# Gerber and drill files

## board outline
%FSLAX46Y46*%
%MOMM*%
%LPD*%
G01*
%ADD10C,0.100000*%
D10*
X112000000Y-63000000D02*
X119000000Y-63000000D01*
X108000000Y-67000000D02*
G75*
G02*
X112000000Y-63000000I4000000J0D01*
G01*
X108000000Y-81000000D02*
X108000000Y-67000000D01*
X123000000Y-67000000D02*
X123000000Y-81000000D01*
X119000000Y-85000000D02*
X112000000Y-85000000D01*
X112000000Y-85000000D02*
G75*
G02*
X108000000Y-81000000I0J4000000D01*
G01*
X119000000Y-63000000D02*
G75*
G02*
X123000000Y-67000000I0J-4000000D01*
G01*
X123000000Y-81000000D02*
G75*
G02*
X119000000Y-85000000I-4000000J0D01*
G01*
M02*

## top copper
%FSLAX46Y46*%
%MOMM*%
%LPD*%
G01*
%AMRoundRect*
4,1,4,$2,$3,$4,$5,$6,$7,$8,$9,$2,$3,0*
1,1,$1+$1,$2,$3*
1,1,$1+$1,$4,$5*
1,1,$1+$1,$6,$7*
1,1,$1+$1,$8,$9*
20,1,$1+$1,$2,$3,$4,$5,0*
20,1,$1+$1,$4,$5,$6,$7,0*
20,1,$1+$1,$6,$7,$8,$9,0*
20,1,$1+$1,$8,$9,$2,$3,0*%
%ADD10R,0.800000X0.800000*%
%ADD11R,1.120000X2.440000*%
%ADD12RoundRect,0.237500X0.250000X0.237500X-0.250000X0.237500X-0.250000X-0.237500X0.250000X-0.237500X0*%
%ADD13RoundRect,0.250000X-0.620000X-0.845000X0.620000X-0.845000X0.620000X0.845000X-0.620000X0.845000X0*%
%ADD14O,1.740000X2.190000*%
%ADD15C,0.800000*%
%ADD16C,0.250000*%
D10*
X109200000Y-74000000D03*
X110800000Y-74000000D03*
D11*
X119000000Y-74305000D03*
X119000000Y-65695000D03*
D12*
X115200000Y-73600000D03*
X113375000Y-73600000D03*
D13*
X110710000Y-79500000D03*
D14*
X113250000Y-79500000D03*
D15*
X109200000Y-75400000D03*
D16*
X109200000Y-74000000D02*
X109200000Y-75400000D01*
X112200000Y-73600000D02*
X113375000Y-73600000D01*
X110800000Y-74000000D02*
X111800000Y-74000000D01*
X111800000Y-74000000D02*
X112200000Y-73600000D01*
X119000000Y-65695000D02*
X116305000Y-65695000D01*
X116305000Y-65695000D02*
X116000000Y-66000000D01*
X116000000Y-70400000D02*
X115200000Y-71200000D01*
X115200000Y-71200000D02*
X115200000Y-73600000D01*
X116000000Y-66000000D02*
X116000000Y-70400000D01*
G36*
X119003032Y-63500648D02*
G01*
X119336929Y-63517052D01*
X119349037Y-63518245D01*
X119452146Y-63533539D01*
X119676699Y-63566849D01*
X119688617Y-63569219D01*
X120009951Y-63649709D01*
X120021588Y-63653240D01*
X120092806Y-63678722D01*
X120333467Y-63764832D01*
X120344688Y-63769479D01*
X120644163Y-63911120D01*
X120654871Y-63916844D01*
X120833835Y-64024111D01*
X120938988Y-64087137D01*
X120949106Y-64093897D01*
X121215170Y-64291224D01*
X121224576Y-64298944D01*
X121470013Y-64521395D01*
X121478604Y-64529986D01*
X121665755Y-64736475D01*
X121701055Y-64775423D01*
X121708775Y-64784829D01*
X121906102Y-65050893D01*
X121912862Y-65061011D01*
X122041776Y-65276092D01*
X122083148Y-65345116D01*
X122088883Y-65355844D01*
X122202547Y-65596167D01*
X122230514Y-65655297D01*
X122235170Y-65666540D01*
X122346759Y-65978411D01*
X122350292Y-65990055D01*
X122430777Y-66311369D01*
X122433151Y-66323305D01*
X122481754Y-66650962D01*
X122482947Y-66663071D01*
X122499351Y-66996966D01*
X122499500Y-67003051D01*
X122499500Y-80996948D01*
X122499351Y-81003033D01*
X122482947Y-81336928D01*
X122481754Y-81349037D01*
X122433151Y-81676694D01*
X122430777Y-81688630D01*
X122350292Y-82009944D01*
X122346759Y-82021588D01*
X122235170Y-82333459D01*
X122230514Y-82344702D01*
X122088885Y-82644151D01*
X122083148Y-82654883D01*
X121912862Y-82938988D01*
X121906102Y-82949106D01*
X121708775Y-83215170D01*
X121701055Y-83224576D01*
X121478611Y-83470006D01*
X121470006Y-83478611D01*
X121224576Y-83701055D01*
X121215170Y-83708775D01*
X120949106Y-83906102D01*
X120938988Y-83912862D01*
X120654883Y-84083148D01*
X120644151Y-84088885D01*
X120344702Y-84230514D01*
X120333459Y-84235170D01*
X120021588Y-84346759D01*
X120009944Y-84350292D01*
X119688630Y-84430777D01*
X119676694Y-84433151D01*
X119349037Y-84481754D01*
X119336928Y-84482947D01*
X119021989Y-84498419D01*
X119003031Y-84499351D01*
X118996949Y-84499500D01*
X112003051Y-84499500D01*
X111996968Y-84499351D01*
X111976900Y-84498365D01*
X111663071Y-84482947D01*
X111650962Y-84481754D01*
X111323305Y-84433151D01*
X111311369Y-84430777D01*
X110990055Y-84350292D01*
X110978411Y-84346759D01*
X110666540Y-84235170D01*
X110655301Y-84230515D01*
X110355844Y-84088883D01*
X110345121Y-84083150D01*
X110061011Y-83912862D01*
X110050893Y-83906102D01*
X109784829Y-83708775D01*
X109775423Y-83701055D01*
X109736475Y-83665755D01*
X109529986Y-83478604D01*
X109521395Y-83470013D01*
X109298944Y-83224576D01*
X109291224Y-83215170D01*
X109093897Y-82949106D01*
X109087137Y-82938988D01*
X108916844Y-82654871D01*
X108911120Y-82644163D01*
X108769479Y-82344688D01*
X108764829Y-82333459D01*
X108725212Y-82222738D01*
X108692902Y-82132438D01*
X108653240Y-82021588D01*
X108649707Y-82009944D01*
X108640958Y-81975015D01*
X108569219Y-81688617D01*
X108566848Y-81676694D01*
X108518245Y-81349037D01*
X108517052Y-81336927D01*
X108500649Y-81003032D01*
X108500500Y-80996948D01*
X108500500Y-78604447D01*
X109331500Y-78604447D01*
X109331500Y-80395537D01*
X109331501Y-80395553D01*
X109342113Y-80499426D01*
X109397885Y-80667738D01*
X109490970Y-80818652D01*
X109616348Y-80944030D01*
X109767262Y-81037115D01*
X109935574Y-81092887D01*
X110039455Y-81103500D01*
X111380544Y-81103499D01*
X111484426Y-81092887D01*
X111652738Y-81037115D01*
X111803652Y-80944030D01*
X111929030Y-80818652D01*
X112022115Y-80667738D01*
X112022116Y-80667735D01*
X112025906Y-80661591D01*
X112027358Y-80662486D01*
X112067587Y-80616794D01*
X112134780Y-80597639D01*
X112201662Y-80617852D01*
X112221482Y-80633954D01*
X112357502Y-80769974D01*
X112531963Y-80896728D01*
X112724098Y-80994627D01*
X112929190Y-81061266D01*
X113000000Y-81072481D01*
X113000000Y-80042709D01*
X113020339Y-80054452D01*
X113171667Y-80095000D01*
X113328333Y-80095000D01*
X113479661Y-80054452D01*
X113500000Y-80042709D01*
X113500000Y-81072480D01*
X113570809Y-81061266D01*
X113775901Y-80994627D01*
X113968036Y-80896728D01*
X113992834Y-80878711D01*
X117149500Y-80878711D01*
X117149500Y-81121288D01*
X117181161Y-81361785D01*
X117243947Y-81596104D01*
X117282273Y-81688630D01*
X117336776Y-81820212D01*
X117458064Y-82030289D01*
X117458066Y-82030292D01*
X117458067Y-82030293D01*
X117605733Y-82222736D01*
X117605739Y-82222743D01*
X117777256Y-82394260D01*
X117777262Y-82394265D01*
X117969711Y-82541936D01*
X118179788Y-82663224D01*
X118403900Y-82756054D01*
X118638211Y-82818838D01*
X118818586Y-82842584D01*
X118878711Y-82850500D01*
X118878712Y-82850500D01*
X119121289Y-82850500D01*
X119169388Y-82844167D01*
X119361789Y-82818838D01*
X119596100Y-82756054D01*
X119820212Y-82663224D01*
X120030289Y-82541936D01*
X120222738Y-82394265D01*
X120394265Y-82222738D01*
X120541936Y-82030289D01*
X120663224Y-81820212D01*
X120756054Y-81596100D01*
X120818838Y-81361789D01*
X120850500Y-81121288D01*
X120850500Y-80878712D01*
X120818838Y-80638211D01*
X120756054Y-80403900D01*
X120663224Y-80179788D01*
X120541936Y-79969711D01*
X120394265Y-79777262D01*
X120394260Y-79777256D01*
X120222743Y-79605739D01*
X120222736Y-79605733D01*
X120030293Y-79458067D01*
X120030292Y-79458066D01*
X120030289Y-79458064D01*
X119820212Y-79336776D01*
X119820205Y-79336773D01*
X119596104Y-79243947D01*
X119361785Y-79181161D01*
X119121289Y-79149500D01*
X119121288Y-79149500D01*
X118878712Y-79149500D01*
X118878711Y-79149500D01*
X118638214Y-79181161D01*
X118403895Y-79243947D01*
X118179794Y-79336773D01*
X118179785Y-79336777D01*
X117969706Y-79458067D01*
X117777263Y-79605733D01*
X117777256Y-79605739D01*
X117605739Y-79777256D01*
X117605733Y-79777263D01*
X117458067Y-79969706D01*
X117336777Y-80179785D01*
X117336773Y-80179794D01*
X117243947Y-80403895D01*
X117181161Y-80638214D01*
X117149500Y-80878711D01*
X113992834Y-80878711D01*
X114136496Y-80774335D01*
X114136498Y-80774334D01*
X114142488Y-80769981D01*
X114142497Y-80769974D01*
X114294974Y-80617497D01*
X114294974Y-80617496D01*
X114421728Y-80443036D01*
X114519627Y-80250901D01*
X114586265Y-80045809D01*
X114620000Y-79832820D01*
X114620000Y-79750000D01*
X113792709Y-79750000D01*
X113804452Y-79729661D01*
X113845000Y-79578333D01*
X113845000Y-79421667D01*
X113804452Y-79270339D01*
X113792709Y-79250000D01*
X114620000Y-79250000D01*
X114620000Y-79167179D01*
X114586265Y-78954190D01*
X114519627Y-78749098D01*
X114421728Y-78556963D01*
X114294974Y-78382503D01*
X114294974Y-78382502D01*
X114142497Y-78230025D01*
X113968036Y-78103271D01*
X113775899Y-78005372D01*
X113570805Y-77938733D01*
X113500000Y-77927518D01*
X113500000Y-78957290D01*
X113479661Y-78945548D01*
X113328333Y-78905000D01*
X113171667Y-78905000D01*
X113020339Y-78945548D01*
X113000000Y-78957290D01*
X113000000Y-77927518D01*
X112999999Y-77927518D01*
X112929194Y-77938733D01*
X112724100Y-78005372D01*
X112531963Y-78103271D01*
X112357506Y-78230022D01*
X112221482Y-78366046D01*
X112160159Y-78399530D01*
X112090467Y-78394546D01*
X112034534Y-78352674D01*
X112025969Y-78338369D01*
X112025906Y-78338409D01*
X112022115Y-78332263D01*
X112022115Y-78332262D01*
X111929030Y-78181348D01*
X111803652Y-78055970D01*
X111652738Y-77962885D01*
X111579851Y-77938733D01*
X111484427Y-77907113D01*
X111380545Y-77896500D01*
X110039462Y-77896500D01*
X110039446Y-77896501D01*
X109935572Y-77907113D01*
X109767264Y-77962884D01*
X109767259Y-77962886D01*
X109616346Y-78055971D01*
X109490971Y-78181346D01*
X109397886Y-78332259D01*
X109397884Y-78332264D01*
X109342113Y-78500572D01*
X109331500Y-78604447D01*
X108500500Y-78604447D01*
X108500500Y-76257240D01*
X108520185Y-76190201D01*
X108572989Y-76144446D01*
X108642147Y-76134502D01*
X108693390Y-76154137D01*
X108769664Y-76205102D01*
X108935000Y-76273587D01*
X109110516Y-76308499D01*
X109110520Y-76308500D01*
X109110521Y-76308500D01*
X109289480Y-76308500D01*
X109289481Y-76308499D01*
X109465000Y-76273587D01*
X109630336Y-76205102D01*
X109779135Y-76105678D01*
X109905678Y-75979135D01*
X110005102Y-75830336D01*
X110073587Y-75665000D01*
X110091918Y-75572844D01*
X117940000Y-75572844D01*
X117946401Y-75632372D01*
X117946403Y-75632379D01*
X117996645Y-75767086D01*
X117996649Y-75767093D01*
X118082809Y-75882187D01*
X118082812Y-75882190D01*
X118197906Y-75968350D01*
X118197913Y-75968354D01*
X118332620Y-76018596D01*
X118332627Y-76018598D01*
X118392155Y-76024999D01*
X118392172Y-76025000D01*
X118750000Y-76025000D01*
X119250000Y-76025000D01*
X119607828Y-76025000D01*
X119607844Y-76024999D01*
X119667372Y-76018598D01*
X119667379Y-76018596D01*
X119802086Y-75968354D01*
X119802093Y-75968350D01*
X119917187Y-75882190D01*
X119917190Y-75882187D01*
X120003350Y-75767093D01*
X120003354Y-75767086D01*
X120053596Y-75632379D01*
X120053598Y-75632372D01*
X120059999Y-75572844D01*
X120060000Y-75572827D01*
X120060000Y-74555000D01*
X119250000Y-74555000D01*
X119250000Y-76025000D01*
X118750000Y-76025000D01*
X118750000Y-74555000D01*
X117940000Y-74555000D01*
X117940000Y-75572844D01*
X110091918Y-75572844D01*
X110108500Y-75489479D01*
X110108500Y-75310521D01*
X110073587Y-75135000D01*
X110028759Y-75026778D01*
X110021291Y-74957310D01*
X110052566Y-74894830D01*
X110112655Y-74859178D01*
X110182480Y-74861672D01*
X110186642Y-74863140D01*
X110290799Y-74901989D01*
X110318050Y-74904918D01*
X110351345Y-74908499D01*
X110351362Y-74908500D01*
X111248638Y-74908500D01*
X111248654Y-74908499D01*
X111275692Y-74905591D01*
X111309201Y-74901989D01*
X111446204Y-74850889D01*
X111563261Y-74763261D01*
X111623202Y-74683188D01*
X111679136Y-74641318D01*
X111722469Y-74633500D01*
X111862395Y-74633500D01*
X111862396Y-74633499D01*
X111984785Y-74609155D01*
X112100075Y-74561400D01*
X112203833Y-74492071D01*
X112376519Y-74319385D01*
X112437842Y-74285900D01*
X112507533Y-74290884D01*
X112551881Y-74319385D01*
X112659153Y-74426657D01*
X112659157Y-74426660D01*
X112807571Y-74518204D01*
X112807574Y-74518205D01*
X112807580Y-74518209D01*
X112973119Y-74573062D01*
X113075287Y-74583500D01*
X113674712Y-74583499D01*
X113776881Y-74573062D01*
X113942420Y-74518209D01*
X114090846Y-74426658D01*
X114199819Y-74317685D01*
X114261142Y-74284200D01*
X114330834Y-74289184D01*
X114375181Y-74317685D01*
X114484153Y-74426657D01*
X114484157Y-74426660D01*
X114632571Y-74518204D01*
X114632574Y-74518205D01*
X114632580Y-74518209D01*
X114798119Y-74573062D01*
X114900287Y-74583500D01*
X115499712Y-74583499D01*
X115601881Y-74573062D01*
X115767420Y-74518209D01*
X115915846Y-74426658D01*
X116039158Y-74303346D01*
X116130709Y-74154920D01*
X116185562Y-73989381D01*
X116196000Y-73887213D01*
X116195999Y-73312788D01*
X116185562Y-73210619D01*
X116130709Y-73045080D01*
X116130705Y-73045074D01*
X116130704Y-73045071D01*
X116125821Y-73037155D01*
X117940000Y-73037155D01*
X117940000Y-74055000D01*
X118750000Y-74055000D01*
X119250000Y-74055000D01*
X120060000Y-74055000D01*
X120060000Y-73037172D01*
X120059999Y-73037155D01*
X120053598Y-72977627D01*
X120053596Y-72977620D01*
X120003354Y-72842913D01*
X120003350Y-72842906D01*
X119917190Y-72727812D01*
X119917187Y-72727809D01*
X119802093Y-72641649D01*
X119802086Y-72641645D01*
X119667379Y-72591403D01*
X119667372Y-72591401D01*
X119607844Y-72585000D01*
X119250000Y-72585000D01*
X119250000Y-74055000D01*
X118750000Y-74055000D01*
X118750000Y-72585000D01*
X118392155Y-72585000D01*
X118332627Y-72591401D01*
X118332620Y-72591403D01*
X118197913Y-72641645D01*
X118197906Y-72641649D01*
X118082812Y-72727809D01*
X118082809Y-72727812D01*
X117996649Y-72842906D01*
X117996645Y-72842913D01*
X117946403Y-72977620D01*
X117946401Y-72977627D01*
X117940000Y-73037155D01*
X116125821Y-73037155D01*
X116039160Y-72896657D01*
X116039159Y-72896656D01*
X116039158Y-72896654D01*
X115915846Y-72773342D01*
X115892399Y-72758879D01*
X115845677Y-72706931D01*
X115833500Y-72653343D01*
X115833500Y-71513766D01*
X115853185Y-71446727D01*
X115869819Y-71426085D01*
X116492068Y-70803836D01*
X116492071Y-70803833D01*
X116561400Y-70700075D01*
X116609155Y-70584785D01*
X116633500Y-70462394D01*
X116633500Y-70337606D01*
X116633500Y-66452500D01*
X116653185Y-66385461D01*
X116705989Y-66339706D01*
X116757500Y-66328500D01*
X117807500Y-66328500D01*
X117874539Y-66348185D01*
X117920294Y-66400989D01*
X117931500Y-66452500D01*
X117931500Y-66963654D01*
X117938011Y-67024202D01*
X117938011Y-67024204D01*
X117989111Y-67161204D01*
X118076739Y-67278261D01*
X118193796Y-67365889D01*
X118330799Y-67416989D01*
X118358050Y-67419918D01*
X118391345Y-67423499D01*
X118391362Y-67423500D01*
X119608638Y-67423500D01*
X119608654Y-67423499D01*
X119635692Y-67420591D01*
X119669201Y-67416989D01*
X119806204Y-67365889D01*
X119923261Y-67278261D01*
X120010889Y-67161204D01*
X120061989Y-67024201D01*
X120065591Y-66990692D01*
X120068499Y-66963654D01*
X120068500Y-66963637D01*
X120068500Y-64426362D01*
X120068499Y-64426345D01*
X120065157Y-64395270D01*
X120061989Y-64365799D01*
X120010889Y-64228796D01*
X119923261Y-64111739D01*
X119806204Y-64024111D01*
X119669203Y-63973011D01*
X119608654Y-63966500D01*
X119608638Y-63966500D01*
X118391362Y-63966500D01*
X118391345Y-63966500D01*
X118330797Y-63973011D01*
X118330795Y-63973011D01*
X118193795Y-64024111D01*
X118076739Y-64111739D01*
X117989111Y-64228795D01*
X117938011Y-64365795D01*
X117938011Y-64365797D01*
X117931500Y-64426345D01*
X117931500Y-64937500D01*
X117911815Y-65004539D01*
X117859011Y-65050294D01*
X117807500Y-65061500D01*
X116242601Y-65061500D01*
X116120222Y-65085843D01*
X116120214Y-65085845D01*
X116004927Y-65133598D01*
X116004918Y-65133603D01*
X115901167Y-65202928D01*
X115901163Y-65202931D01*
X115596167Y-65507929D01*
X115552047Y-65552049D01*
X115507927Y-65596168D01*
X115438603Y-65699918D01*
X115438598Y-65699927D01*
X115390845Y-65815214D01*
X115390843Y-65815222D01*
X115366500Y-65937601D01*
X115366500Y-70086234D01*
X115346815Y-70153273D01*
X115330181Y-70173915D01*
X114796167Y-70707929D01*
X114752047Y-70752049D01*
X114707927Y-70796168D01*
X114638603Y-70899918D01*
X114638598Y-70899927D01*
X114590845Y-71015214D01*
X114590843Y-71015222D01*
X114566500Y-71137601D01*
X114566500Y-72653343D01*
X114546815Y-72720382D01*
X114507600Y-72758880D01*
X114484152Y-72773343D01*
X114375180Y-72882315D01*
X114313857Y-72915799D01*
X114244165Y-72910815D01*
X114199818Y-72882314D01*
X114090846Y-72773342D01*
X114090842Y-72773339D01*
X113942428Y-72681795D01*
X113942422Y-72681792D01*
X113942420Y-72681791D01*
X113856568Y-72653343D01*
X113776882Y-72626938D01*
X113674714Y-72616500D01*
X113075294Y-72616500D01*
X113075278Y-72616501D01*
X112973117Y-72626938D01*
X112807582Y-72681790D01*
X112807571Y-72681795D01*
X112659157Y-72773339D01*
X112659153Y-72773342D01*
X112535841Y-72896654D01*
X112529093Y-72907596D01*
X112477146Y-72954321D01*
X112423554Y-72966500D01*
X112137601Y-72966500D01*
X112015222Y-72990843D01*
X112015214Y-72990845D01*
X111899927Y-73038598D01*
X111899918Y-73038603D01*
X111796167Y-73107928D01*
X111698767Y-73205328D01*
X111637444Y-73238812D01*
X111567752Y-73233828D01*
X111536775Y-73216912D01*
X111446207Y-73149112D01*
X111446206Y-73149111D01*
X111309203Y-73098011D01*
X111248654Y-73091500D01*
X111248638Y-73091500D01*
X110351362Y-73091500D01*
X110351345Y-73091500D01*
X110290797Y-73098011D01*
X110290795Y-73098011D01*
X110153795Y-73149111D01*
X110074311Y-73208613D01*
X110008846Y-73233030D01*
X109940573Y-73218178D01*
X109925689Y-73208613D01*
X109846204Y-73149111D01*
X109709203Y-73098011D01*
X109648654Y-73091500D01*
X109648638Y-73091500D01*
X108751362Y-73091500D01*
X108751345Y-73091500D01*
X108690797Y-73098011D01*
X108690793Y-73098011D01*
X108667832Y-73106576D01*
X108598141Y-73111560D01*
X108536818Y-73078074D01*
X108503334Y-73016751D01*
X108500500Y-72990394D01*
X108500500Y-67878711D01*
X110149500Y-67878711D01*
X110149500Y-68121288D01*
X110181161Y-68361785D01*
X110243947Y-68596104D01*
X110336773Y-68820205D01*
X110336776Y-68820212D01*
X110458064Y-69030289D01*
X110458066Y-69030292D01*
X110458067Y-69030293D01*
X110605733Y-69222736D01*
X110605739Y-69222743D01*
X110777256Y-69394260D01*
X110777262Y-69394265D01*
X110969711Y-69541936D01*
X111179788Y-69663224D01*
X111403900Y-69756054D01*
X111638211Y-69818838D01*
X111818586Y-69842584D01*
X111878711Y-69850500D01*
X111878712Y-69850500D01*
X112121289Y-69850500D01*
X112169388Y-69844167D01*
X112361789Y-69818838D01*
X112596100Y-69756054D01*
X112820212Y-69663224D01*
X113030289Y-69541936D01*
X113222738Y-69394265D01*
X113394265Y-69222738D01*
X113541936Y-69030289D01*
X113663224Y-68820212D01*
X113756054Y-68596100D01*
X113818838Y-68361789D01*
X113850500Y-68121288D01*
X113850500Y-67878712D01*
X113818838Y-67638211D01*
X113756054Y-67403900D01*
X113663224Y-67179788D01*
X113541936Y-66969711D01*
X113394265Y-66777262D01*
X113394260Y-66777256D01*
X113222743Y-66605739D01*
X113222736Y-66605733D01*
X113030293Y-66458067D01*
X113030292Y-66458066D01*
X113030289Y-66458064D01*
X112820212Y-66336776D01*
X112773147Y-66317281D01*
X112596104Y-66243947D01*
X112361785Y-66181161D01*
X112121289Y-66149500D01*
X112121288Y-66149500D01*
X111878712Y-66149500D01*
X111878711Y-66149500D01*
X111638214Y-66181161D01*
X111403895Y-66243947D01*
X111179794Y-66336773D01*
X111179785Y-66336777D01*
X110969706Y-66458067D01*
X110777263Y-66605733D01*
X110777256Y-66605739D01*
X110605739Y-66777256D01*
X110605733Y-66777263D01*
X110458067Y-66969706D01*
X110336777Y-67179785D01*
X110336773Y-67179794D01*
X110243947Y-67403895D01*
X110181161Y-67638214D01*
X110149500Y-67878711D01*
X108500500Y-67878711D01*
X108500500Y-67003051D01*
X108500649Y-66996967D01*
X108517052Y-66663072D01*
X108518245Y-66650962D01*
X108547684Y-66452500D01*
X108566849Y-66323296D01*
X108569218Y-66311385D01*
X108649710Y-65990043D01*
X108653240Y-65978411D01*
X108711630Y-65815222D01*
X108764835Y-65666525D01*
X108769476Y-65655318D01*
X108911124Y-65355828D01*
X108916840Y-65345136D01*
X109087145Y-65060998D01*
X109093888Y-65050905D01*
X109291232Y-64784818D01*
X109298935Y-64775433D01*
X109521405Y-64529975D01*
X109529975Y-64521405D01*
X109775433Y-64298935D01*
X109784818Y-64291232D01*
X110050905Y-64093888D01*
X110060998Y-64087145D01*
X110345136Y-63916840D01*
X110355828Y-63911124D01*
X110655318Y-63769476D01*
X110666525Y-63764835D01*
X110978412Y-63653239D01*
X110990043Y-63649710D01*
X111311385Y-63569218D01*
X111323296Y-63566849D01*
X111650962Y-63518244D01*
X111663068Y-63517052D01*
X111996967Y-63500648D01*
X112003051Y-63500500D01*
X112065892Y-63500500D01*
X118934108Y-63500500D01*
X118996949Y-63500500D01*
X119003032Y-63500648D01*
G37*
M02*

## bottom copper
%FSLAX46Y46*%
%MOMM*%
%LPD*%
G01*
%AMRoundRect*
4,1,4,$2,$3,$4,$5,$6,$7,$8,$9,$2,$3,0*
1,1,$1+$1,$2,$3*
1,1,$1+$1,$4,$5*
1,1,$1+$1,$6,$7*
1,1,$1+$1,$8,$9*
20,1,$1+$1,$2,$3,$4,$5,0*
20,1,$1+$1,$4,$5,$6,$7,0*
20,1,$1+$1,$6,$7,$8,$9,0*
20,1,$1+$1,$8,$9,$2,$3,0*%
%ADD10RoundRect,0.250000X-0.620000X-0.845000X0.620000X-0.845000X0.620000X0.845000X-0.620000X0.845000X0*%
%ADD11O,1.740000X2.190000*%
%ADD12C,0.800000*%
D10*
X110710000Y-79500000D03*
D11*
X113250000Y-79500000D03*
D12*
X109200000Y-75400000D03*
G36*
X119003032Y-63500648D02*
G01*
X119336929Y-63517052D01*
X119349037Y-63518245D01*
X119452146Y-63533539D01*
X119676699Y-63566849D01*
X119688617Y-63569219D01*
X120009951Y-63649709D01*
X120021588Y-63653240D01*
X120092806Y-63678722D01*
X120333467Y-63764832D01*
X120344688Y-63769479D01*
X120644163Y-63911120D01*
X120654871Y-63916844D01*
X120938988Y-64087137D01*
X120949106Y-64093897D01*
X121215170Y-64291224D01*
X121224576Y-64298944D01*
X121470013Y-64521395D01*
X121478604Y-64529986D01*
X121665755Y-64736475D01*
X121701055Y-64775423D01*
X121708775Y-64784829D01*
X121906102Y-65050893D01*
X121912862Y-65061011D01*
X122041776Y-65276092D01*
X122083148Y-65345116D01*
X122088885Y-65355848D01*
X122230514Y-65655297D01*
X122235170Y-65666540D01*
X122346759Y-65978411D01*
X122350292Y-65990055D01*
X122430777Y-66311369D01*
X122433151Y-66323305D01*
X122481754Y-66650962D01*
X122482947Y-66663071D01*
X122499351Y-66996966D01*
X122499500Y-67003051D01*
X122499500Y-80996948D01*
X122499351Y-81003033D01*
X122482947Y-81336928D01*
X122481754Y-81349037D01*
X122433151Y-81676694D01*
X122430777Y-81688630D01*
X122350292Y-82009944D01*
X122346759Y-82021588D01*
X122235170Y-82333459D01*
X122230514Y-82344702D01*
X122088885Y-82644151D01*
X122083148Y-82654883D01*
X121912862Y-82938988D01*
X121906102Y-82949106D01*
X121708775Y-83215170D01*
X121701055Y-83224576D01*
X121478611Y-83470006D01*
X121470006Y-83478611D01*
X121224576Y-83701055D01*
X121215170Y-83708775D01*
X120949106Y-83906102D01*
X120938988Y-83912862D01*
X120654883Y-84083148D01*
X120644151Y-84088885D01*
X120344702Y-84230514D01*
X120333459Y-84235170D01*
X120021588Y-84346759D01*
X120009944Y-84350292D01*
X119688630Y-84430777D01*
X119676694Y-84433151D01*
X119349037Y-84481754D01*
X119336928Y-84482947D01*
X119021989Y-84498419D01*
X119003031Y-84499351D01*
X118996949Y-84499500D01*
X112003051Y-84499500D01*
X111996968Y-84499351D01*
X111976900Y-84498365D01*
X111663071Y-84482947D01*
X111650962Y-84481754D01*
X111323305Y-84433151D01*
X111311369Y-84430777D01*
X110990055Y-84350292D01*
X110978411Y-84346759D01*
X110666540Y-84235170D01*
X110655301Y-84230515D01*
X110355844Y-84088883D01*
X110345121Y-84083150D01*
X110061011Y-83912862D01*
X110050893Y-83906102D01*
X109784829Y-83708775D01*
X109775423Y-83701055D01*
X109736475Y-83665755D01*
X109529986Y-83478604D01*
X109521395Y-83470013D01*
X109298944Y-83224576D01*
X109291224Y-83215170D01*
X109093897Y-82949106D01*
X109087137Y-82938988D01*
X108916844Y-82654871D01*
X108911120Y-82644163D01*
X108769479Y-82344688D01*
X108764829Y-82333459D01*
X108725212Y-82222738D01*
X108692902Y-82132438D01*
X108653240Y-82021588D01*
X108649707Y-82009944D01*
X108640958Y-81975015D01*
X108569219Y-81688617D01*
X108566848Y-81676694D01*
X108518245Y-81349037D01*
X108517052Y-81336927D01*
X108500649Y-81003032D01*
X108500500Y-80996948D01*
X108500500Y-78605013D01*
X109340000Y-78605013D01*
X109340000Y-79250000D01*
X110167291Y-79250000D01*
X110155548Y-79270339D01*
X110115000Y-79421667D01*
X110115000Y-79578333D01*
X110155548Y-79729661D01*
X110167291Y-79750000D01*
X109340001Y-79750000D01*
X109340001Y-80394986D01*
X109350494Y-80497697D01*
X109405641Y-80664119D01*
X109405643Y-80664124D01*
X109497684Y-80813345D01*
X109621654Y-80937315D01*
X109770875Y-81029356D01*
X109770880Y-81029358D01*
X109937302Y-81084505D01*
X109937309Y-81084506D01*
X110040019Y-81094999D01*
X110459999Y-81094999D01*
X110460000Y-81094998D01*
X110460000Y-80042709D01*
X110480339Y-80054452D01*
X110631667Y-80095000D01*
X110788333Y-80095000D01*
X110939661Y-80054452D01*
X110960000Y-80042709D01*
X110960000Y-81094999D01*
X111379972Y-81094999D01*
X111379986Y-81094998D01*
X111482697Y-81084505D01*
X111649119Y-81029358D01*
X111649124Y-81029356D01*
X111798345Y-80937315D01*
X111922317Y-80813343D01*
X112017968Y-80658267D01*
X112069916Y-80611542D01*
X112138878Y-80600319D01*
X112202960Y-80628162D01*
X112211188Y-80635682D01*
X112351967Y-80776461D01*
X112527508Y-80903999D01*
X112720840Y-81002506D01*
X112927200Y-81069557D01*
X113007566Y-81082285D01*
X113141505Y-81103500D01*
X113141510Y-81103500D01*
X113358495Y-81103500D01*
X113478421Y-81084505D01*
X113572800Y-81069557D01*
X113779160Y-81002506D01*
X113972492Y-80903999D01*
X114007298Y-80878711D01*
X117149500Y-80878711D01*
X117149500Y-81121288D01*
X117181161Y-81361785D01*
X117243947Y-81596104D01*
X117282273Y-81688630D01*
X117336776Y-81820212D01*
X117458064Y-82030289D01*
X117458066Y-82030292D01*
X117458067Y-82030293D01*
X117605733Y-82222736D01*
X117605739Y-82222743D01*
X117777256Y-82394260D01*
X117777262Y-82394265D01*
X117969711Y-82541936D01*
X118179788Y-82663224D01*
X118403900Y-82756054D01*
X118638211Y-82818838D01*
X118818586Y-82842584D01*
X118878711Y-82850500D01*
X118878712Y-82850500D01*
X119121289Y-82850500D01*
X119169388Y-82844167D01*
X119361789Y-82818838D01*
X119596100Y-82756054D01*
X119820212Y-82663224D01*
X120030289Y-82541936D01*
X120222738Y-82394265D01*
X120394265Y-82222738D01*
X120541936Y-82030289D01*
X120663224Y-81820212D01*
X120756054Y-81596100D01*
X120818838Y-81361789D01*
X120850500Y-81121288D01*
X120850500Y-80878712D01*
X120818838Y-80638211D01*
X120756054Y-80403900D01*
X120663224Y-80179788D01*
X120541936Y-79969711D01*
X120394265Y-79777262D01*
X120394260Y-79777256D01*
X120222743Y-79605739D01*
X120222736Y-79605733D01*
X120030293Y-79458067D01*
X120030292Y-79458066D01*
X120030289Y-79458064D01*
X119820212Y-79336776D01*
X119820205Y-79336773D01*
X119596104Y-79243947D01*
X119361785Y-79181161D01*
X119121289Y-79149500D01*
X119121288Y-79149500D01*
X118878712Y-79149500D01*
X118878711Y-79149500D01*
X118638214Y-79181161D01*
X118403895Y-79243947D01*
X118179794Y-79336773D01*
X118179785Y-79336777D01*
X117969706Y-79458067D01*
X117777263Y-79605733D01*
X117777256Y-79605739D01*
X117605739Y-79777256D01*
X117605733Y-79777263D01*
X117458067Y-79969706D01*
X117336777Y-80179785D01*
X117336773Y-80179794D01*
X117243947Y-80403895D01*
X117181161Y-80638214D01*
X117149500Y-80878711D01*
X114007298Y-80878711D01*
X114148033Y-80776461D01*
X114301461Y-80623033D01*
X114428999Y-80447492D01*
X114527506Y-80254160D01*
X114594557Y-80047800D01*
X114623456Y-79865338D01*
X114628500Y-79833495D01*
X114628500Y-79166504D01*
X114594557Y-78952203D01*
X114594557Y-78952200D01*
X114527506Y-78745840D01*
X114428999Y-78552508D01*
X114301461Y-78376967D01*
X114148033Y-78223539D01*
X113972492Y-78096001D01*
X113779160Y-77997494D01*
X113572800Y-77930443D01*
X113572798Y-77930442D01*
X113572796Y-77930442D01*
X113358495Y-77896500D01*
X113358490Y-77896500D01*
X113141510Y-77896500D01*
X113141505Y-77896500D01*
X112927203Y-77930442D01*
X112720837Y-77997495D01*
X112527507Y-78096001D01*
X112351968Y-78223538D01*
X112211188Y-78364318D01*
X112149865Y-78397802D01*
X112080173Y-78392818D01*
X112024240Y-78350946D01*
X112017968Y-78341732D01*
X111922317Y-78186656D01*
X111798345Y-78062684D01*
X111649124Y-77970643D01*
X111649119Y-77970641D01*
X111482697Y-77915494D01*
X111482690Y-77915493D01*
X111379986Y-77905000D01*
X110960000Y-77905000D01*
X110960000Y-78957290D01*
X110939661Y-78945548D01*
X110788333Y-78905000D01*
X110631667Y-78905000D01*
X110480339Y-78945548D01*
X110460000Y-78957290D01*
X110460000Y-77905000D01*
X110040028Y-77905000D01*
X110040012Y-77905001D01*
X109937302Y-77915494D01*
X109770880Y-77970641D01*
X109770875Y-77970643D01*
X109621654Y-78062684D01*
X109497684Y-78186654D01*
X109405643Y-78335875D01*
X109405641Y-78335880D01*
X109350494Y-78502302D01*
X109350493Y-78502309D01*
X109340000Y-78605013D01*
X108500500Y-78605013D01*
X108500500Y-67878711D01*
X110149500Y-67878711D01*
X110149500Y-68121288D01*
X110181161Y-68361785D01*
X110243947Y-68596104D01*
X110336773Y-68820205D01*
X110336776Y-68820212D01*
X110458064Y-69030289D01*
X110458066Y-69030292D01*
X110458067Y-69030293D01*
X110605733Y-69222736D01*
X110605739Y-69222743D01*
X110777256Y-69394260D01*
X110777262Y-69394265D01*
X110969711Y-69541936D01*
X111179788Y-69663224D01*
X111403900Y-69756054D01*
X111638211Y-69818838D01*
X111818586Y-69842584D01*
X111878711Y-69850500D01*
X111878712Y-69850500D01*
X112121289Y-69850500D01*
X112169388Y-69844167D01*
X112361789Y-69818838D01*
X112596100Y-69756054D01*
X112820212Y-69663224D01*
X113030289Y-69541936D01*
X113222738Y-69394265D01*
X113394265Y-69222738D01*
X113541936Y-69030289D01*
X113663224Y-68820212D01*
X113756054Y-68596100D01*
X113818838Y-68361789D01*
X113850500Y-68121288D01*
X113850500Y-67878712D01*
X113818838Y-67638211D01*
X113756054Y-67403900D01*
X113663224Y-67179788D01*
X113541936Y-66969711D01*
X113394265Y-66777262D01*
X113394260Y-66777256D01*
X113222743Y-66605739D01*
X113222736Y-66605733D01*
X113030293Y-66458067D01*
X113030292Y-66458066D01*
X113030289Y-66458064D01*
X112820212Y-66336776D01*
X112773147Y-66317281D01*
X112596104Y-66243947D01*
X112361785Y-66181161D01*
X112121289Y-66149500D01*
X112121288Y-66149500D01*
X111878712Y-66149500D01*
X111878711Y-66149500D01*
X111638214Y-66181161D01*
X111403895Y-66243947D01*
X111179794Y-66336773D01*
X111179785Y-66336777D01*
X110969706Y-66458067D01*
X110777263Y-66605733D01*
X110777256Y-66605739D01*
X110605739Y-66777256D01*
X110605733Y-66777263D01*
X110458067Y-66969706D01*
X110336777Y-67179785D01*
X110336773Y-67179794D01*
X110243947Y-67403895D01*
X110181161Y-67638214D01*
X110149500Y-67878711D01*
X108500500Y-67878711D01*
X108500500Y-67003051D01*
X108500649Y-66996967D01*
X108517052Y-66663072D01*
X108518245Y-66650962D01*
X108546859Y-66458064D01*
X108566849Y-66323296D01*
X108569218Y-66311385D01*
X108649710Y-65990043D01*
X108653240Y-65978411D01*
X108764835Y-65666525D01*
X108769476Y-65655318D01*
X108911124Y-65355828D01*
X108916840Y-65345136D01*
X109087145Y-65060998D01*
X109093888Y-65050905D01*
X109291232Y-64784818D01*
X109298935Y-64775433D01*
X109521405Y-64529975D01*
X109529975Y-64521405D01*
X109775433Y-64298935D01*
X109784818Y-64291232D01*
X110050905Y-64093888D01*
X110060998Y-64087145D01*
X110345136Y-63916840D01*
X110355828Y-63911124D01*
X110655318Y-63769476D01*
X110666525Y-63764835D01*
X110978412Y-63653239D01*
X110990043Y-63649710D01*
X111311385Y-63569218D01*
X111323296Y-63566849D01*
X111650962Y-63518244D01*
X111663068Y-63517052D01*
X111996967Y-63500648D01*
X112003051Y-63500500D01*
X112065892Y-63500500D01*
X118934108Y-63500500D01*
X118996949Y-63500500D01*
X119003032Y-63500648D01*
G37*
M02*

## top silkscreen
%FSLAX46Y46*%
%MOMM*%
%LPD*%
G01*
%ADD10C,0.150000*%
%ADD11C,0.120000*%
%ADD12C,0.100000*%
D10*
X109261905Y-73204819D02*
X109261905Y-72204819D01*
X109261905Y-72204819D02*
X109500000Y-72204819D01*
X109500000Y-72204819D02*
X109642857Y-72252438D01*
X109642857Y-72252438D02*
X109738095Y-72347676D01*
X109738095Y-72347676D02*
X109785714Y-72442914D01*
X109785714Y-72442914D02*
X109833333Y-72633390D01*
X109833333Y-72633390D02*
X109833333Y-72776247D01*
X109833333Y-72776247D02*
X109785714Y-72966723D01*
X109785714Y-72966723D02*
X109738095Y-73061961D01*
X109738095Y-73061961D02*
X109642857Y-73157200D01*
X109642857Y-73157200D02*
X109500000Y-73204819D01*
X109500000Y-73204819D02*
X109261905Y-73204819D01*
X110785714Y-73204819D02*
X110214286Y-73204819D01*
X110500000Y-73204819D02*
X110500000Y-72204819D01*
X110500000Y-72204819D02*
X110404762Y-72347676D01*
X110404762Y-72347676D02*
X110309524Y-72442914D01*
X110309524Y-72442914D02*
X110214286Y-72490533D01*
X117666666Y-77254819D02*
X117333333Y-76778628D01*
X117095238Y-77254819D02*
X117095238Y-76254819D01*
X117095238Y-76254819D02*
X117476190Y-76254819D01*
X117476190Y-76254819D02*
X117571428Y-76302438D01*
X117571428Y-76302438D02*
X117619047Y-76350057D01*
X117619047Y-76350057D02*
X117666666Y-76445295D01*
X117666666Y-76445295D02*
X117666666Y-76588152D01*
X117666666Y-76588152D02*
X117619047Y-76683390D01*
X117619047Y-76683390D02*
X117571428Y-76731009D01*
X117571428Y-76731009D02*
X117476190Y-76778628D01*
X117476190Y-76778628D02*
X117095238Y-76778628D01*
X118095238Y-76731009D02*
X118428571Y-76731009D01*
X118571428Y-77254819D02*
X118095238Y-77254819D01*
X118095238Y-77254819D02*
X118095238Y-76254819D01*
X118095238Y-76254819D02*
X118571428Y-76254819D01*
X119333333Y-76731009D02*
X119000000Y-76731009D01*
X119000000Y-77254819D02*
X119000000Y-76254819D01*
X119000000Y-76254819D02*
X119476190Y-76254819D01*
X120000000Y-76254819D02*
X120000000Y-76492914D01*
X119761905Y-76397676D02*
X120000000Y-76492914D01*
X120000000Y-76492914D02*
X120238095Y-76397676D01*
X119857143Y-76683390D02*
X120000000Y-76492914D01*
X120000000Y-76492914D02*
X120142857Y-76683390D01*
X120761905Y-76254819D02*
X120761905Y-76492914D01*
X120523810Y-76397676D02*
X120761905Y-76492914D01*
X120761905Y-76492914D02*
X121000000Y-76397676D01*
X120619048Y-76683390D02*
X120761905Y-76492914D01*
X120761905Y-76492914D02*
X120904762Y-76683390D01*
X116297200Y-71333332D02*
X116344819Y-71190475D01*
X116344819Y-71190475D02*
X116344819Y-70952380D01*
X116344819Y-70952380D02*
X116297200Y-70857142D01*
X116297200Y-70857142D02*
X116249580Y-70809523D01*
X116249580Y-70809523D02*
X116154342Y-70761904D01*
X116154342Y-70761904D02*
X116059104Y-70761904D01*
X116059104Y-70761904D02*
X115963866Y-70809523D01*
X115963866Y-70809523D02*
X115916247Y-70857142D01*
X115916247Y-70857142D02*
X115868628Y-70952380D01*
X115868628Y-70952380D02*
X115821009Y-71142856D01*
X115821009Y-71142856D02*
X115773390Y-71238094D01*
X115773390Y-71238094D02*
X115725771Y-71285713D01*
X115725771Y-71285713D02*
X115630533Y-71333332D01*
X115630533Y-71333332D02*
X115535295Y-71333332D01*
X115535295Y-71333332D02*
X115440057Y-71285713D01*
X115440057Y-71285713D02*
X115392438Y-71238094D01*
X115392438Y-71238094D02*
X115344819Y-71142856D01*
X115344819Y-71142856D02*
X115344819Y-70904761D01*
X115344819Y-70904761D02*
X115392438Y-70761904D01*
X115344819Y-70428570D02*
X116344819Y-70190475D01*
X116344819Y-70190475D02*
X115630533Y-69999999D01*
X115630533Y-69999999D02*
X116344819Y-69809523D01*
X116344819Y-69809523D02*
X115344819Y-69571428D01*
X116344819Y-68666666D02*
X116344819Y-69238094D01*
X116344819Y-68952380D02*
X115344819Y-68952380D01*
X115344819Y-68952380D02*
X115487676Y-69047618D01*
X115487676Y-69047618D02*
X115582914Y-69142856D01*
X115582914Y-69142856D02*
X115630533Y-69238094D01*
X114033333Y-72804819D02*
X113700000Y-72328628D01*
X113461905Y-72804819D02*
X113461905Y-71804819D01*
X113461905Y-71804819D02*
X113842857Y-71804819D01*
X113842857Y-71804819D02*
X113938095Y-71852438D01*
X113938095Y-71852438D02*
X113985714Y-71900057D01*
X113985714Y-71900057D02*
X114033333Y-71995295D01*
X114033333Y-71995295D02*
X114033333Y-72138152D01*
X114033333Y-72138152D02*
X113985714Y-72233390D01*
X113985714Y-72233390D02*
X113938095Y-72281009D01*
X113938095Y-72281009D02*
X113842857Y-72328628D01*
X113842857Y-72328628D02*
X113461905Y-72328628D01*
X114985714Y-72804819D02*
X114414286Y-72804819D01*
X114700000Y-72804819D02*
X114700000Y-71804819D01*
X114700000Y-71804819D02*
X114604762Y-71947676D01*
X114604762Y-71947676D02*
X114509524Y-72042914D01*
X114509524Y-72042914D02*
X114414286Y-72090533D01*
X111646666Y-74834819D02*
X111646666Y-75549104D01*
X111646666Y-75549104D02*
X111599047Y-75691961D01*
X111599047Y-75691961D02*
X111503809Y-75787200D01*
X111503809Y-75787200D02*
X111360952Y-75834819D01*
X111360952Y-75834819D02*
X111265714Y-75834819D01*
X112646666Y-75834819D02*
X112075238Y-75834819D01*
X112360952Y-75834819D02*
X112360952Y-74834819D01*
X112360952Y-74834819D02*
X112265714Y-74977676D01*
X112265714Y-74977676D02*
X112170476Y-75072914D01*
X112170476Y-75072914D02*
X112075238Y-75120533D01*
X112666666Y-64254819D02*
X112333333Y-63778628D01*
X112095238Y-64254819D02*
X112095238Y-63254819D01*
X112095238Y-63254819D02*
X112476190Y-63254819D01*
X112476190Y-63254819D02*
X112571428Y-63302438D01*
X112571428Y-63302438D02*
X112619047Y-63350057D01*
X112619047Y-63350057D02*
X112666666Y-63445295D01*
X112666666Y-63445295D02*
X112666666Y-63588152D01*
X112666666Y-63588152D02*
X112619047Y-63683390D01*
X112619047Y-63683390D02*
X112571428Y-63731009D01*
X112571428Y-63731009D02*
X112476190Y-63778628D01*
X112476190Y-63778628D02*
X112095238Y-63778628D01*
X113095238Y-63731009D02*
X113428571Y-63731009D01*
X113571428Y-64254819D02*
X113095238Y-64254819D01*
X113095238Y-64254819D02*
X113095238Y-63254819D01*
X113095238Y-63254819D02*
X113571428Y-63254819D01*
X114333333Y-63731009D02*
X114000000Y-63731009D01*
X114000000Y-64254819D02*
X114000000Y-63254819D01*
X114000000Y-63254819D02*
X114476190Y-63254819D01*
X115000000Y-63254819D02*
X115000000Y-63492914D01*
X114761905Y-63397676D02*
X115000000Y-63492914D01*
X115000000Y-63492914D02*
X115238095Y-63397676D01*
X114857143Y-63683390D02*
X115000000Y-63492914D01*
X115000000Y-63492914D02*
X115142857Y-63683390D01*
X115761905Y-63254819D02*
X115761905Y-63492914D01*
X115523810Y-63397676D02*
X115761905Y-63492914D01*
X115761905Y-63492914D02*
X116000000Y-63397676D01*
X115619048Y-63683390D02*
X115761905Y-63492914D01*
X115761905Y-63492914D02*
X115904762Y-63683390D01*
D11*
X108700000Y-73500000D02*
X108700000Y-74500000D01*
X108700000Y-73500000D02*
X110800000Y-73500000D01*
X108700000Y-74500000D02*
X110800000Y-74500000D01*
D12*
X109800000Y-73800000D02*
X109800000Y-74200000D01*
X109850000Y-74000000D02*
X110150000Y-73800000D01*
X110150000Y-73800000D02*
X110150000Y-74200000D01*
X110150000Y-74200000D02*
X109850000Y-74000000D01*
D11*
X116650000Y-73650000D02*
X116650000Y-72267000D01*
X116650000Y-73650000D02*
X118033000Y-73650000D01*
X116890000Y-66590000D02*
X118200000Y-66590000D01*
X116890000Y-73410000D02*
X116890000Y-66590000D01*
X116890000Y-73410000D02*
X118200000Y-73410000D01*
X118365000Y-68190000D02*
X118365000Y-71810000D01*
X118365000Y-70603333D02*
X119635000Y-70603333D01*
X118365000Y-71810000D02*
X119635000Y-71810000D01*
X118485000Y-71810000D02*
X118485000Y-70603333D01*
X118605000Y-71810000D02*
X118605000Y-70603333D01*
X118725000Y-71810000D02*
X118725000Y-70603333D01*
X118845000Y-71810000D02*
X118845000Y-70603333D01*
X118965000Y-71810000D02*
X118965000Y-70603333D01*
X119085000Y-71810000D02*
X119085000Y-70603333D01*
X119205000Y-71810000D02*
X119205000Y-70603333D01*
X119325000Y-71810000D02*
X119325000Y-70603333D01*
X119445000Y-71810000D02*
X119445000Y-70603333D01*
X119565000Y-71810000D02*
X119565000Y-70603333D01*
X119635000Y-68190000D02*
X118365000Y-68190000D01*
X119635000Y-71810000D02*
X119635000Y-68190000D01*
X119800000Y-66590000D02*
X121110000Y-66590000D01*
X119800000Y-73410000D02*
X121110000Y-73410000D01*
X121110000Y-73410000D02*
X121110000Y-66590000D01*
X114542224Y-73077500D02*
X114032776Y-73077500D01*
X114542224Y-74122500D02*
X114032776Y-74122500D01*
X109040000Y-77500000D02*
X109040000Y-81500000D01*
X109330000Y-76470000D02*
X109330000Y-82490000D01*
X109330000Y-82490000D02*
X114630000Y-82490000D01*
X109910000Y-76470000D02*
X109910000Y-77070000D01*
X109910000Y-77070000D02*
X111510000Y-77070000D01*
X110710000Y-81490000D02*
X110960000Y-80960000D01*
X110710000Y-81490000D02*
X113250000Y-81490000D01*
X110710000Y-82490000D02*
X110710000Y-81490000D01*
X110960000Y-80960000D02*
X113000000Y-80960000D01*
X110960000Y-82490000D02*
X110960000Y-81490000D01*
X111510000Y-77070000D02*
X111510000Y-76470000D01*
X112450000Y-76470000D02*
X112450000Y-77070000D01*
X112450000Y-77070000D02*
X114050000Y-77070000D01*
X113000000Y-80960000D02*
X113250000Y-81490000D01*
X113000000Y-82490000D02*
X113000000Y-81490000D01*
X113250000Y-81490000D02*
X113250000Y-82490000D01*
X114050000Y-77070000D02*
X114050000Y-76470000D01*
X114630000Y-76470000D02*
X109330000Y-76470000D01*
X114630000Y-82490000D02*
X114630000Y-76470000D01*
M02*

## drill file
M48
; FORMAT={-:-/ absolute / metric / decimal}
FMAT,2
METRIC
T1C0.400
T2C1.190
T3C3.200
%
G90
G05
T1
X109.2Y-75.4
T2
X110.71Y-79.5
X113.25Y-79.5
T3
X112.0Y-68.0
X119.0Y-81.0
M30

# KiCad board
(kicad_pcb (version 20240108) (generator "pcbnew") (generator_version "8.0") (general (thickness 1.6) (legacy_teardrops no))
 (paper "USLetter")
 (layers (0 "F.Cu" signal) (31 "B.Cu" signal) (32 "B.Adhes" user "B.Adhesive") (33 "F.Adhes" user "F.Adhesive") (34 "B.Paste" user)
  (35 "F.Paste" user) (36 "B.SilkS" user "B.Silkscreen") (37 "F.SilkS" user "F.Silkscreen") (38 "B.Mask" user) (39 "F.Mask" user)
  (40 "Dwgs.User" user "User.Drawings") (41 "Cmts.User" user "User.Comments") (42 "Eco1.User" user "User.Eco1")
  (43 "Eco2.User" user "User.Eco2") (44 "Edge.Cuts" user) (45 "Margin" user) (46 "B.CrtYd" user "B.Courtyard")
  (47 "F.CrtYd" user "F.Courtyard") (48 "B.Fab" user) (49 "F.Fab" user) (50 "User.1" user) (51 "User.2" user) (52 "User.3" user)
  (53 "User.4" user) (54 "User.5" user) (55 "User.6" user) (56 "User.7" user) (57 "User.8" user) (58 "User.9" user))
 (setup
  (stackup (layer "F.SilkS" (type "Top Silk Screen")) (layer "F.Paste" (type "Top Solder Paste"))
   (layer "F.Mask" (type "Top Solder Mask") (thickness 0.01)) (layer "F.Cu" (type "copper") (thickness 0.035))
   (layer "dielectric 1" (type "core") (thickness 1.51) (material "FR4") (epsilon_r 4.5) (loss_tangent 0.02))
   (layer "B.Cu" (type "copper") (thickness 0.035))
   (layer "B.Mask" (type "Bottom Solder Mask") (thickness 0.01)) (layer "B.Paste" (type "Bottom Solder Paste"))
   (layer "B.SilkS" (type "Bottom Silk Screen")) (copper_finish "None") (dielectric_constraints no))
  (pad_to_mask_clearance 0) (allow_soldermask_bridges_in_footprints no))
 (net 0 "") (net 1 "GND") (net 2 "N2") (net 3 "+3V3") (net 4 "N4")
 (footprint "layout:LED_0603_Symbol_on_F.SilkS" (layer "F.Cu") (at 110 74)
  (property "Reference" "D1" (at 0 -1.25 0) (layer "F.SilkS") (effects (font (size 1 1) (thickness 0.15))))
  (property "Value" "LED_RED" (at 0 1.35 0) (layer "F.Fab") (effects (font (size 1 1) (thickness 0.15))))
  (fp_line (start -1.3 -0.5) (end -1.3 0.5) (stroke (width 0.12) (type solid)) (layer "F.SilkS"))
  (fp_line (start -1.3 -0.5) (end 0.8 -0.5) (stroke (width 0.12) (type solid)) (layer "F.SilkS"))
  (fp_line (start -1.3 0.5) (end 0.8 0.5) (stroke (width 0.12) (type solid)) (layer "F.SilkS"))
  (fp_line (start -0.2 -0.2) (end -0.2 0.2) (stroke (width 0.1) (type solid)) (layer "F.SilkS"))
  (fp_line (start -0.15 0) (end 0.15 -0.2) (stroke (width 0.1) (type solid)) (layer "F.SilkS"))
  (fp_line (start 0.15 -0.2) (end 0.15 0.2) (stroke (width 0.1) (type solid)) (layer "F.SilkS"))
  (fp_line (start 0.15 0.2) (end -0.15 0) (stroke (width 0.1) (type solid)) (layer "F.SilkS"))
  (pad "1" smd rect (at -0.8 0 180) (size 0.8 0.8) (layers "F.Cu" "F.Paste" "F.Mask") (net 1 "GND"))
  (pad "2" smd rect (at 0.8 0 180) (size 0.8 0.8) (layers "F.Cu" "F.Paste" "F.Mask") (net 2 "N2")))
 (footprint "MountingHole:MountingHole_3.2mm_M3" (layer "F.Cu") (at 119 81)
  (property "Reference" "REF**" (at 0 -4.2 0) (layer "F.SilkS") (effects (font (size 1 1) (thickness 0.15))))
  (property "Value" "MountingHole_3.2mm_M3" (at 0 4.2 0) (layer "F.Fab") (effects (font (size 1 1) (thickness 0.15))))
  (pad "" np_thru_hole circle (at 0 0) (size 3.2 3.2) (drill 3.2) (layers "*.Cu" "*.Mask")))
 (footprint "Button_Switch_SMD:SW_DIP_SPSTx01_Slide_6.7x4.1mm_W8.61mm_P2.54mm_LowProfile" (layer "F.Cu") (at 119 70 90)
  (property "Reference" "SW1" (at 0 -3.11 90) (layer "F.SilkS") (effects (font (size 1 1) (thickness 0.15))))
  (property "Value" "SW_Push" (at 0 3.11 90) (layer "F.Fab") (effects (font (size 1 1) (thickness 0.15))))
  (fp_line (start -3.65 -2.35) (end -2.267 -2.35) (stroke (width 0.12) (type solid)) (layer "F.SilkS"))
  (fp_line (start -3.65 -2.35) (end -3.65 -0.967) (stroke (width 0.12) (type solid)) (layer "F.SilkS"))
  (fp_line (start 3.41 -2.11) (end 3.41 -0.8) (stroke (width 0.12) (type solid)) (layer "F.SilkS"))
  (fp_line (start -3.41 -2.11) (end 3.41 -2.11) (stroke (width 0.12) (type solid)) (layer "F.SilkS"))
  (fp_line (start -3.41 -2.11) (end -3.41 -0.8) (stroke (width 0.12) (type solid)) (layer "F.SilkS"))
  (fp_line (start 1.81 -0.635) (end -1.81 -0.635) (stroke (width 0.12) (type solid)) (layer "F.SilkS"))
  (fp_line (start -0.603333 -0.635) (end -0.603333 0.635) (stroke (width 0.12) (type solid)) (layer "F.SilkS"))
  (fp_line (start -1.81 -0.635) (end -1.81 0.635) (stroke (width 0.12) (type solid)) (layer "F.SilkS"))
  (fp_line (start -1.81 -0.515) (end -0.603333 -0.515) (stroke (width 0.12) (type solid)) (layer "F.SilkS"))
  (fp_line (start -1.81 -0.395) (end -0.603333 -0.395) (stroke (width 0.12) (type solid)) (layer "F.SilkS"))
  (fp_line (start -1.81 -0.275) (end -0.603333 -0.275) (stroke (width 0.12) (type solid)) (layer "F.SilkS"))
  (fp_line (start -1.81 -0.155) (end -0.603333 -0.155) (stroke (width 0.12) (type solid)) (layer "F.SilkS"))
  (fp_line (start -1.81 -0.035) (end -0.603333 -0.035) (stroke (width 0.12) (type solid)) (layer "F.SilkS"))
  (fp_line (start -1.81 0.085) (end -0.603333 0.085) (stroke (width 0.12) (type solid)) (layer "F.SilkS"))
  (fp_line (start -1.81 0.205) (end -0.603333 0.205) (stroke (width 0.12) (type solid)) (layer "F.SilkS"))
  (fp_line (start -1.81 0.325) (end -0.603333 0.325) (stroke (width 0.12) (type solid)) (layer "F.SilkS"))
  (fp_line (start -1.81 0.445) (end -0.603333 0.445) (stroke (width 0.12) (type solid)) (layer "F.SilkS"))
  (fp_line (start -1.81 0.565) (end -0.603333 0.565) (stroke (width 0.12) (type solid)) (layer "F.SilkS"))
  (fp_line (start 1.81 0.635) (end 1.81 -0.635) (stroke (width 0.12) (type solid)) (layer "F.SilkS"))
  (fp_line (start -1.81 0.635) (end 1.81 0.635) (stroke (width 0.12) (type solid)) (layer "F.SilkS"))
  (fp_line (start 3.41 0.8) (end 3.41 2.11) (stroke (width 0.12) (type solid)) (layer "F.SilkS"))
  (fp_line (start -3.41 0.8) (end -3.41 2.11) (stroke (width 0.12) (type solid)) (layer "F.SilkS"))
  (fp_line (start -3.41 2.11) (end 3.41 2.11) (stroke (width 0.12) (type solid)) (layer "F.SilkS"))
  (pad "1" smd rect (at -4.305 0 90) (size 2.44 1.12) (layers "F.Cu" "F.Paste" "F.Mask") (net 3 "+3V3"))
  (pad "2" smd rect (at 4.305 0 90) (size 2.44 1.12) (layers "F.Cu" "F.Paste" "F.Mask") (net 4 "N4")))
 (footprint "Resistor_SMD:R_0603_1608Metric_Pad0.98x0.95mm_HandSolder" (layer "F.Cu") (at 114.2875 73.6 180)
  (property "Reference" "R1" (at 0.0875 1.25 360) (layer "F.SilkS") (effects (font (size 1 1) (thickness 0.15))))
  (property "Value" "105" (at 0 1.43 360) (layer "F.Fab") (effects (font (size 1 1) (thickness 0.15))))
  (fp_line (start -0.254724 0.5225) (end 0.254724 0.5225) (stroke (width 0.12) (type solid)) (layer "F.SilkS"))
  (fp_line (start -0.254724 -0.5225) (end 0.254724 -0.5225) (stroke (width 0.12) (type solid)) (layer "F.SilkS"))
  (pad "1" smd roundrect (at -0.9125 0 180) (size 0.975 0.95) (layers "F.Cu" "F.Paste" "F.Mask") (roundrect_rratio 0.25) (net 4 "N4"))
  (pad "2" smd roundrect (at 0.9125 0 180) (size 0.975 0.95) (layers "F.Cu" "F.Paste" "F.Mask") (roundrect_rratio 0.25) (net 2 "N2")))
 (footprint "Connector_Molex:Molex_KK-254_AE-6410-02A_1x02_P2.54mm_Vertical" (layer "F.Cu") (at 110.71 79.5)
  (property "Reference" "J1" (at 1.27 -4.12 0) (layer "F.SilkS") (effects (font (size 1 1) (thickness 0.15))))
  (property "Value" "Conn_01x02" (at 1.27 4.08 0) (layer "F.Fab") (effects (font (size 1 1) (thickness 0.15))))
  (fp_line (start -1.67 -2) (end -1.67 2) (stroke (width 0.12) (type solid)) (layer "F.SilkS"))
  (fp_line (start -1.38 -3.03) (end -1.38 2.99) (stroke (width 0.12) (type solid)) (layer "F.SilkS"))
  (fp_line (start -1.38 2.99) (end 3.92 2.99) (stroke (width 0.12) (type solid)) (layer "F.SilkS"))
  (fp_line (start -0.8 -3.03) (end -0.8 -2.43) (stroke (width 0.12) (type solid)) (layer "F.SilkS"))
  (fp_line (start -0.8 -2.43) (end 0.8 -2.43) (stroke (width 0.12) (type solid)) (layer "F.SilkS"))
  (fp_line (start 0 1.99) (end 0.25 1.46) (stroke (width 0.12) (type solid)) (layer "F.SilkS"))
  (fp_line (start 0 1.99) (end 2.54 1.99) (stroke (width 0.12) (type solid)) (layer "F.SilkS"))
  (fp_line (start 0 2.99) (end 0 1.99) (stroke (width 0.12) (type solid)) (layer "F.SilkS"))
  (fp_line (start 0.25 1.46) (end 2.29 1.46) (stroke (width 0.12) (type solid)) (layer "F.SilkS"))
  (fp_line (start 0.25 2.99) (end 0.25 1.99) (stroke (width 0.12) (type solid)) (layer "F.SilkS"))
  (fp_line (start 0.8 -2.43) (end 0.8 -3.03) (stroke (width 0.12) (type solid)) (layer "F.SilkS"))
  (fp_line (start 1.74 -3.03) (end 1.74 -2.43) (stroke (width 0.12) (type solid)) (layer "F.SilkS"))
  (fp_line (start 1.74 -2.43) (end 3.34 -2.43) (stroke (width 0.12) (type solid)) (layer "F.SilkS"))
  (fp_line (start 2.29 1.46) (end 2.54 1.99) (stroke (width 0.12) (type solid)) (layer "F.SilkS"))
  (fp_line (start 2.29 2.99) (end 2.29 1.99) (stroke (width 0.12) (type solid)) (layer "F.SilkS"))
  (fp_line (start 2.54 1.99) (end 2.54 2.99) (stroke (width 0.12) (type solid)) (layer "F.SilkS"))
  (fp_line (start 3.34 -2.43) (end 3.34 -3.03) (stroke (width 0.12) (type solid)) (layer "F.SilkS"))
  (fp_line (start 3.92 -3.03) (end -1.38 -3.03) (stroke (width 0.12) (type solid)) (layer "F.SilkS"))
  (fp_line (start 3.92 2.99) (end 3.92 -3.03) (stroke (width 0.12) (type solid)) (layer "F.SilkS"))
  (pad "1" thru_hole roundrect (at 0 0) (size 1.74 2.19) (drill 1.19) (layers "*.Cu" "*.Mask") (remove_unused_layers no)
   (roundrect_rratio 0.143678) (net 1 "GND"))
  (pad "2" thru_hole oval (at 2.54 0) (size 1.74 2.19) (drill 1.19) (layers "*.Cu" "*.Mask") (remove_unused_layers no) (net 3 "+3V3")))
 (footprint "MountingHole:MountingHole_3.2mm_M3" (layer "F.Cu") (at 112 68)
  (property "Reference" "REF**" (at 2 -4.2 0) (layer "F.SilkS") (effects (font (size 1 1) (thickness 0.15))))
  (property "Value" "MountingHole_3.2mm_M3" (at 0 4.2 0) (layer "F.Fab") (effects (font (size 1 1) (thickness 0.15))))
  (pad "" np_thru_hole circle (at 0 0) (size 3.2 3.2) (drill 3.2) (layers "*.Cu" "*.Mask")))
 (gr_line (start 112 63) (end 119 63) (stroke (width 0.1) (type default)) (layer "Edge.Cuts"))
 (gr_arc (start 108 67) (mid 109.171573 64.171573) (end 112 63) (stroke (width 0.1) (type default)) (layer "Edge.Cuts"))
 (gr_line (start 108 81) (end 108 67) (stroke (width 0.1) (type default)) (layer "Edge.Cuts"))
 (gr_line (start 123 67) (end 123 81) (stroke (width 0.1) (type default)) (layer "Edge.Cuts"))
 (gr_line (start 119 85) (end 112 85) (stroke (width 0.1) (type default)) (layer "Edge.Cuts"))
 (gr_arc (start 112 85) (mid 109.171573 83.828427) (end 108 81) (stroke (width 0.1) (type default)) (layer "Edge.Cuts"))
 (gr_arc (start 119 63) (mid 121.828427 64.171573) (end 123 67) (stroke (width 0.1) (type default)) (layer "Edge.Cuts"))
 (gr_arc (start 123 81) (mid 121.828427 83.828427) (end 119 85) (stroke (width 0.1) (type default)) (layer "Edge.Cuts"))
 (segment (start 109.2 74) (end 109.2 75.4) (width 0.25) (layer "F.Cu") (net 1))
 (via (at 109.2 75.4) (size 0.8) (drill 0.4) (layers "F.Cu" "B.Cu") (free yes) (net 1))
 (segment (start 112.2 73.6) (end 113.375 73.6) (width 0.25) (layer "F.Cu") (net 2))
 (segment (start 110.8 74) (end 111.8 74) (width 0.25) (layer "F.Cu") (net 2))
 (segment (start 111.8 74) (end 112.2 73.6) (width 0.25) (layer "F.Cu") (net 2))
 (segment (start 119 65.695) (end 116.305 65.695) (width 0.25) (layer "F.Cu") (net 4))
 (segment (start 116.305 65.695) (end 116 66) (width 0.25) (layer "F.Cu") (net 4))
 (segment (start 116 70.4) (end 115.2 71.2) (width 0.25) (layer "F.Cu") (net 4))
 (segment (start 115.2 71.2) (end 115.2 73.6) (width 0.25) (layer "F.Cu") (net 4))
 (segment (start 116 66) (end 116 70.4) (width 0.25) (layer "F.Cu") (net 4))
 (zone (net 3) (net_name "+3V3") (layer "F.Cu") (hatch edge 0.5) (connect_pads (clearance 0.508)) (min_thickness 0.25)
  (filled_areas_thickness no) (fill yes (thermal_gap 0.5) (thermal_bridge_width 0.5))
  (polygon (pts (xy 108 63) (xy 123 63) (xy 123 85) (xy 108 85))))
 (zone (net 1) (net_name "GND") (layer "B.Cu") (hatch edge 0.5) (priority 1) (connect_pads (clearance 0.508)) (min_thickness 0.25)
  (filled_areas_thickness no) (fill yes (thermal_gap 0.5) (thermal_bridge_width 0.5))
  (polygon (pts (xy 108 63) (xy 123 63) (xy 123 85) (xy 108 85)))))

